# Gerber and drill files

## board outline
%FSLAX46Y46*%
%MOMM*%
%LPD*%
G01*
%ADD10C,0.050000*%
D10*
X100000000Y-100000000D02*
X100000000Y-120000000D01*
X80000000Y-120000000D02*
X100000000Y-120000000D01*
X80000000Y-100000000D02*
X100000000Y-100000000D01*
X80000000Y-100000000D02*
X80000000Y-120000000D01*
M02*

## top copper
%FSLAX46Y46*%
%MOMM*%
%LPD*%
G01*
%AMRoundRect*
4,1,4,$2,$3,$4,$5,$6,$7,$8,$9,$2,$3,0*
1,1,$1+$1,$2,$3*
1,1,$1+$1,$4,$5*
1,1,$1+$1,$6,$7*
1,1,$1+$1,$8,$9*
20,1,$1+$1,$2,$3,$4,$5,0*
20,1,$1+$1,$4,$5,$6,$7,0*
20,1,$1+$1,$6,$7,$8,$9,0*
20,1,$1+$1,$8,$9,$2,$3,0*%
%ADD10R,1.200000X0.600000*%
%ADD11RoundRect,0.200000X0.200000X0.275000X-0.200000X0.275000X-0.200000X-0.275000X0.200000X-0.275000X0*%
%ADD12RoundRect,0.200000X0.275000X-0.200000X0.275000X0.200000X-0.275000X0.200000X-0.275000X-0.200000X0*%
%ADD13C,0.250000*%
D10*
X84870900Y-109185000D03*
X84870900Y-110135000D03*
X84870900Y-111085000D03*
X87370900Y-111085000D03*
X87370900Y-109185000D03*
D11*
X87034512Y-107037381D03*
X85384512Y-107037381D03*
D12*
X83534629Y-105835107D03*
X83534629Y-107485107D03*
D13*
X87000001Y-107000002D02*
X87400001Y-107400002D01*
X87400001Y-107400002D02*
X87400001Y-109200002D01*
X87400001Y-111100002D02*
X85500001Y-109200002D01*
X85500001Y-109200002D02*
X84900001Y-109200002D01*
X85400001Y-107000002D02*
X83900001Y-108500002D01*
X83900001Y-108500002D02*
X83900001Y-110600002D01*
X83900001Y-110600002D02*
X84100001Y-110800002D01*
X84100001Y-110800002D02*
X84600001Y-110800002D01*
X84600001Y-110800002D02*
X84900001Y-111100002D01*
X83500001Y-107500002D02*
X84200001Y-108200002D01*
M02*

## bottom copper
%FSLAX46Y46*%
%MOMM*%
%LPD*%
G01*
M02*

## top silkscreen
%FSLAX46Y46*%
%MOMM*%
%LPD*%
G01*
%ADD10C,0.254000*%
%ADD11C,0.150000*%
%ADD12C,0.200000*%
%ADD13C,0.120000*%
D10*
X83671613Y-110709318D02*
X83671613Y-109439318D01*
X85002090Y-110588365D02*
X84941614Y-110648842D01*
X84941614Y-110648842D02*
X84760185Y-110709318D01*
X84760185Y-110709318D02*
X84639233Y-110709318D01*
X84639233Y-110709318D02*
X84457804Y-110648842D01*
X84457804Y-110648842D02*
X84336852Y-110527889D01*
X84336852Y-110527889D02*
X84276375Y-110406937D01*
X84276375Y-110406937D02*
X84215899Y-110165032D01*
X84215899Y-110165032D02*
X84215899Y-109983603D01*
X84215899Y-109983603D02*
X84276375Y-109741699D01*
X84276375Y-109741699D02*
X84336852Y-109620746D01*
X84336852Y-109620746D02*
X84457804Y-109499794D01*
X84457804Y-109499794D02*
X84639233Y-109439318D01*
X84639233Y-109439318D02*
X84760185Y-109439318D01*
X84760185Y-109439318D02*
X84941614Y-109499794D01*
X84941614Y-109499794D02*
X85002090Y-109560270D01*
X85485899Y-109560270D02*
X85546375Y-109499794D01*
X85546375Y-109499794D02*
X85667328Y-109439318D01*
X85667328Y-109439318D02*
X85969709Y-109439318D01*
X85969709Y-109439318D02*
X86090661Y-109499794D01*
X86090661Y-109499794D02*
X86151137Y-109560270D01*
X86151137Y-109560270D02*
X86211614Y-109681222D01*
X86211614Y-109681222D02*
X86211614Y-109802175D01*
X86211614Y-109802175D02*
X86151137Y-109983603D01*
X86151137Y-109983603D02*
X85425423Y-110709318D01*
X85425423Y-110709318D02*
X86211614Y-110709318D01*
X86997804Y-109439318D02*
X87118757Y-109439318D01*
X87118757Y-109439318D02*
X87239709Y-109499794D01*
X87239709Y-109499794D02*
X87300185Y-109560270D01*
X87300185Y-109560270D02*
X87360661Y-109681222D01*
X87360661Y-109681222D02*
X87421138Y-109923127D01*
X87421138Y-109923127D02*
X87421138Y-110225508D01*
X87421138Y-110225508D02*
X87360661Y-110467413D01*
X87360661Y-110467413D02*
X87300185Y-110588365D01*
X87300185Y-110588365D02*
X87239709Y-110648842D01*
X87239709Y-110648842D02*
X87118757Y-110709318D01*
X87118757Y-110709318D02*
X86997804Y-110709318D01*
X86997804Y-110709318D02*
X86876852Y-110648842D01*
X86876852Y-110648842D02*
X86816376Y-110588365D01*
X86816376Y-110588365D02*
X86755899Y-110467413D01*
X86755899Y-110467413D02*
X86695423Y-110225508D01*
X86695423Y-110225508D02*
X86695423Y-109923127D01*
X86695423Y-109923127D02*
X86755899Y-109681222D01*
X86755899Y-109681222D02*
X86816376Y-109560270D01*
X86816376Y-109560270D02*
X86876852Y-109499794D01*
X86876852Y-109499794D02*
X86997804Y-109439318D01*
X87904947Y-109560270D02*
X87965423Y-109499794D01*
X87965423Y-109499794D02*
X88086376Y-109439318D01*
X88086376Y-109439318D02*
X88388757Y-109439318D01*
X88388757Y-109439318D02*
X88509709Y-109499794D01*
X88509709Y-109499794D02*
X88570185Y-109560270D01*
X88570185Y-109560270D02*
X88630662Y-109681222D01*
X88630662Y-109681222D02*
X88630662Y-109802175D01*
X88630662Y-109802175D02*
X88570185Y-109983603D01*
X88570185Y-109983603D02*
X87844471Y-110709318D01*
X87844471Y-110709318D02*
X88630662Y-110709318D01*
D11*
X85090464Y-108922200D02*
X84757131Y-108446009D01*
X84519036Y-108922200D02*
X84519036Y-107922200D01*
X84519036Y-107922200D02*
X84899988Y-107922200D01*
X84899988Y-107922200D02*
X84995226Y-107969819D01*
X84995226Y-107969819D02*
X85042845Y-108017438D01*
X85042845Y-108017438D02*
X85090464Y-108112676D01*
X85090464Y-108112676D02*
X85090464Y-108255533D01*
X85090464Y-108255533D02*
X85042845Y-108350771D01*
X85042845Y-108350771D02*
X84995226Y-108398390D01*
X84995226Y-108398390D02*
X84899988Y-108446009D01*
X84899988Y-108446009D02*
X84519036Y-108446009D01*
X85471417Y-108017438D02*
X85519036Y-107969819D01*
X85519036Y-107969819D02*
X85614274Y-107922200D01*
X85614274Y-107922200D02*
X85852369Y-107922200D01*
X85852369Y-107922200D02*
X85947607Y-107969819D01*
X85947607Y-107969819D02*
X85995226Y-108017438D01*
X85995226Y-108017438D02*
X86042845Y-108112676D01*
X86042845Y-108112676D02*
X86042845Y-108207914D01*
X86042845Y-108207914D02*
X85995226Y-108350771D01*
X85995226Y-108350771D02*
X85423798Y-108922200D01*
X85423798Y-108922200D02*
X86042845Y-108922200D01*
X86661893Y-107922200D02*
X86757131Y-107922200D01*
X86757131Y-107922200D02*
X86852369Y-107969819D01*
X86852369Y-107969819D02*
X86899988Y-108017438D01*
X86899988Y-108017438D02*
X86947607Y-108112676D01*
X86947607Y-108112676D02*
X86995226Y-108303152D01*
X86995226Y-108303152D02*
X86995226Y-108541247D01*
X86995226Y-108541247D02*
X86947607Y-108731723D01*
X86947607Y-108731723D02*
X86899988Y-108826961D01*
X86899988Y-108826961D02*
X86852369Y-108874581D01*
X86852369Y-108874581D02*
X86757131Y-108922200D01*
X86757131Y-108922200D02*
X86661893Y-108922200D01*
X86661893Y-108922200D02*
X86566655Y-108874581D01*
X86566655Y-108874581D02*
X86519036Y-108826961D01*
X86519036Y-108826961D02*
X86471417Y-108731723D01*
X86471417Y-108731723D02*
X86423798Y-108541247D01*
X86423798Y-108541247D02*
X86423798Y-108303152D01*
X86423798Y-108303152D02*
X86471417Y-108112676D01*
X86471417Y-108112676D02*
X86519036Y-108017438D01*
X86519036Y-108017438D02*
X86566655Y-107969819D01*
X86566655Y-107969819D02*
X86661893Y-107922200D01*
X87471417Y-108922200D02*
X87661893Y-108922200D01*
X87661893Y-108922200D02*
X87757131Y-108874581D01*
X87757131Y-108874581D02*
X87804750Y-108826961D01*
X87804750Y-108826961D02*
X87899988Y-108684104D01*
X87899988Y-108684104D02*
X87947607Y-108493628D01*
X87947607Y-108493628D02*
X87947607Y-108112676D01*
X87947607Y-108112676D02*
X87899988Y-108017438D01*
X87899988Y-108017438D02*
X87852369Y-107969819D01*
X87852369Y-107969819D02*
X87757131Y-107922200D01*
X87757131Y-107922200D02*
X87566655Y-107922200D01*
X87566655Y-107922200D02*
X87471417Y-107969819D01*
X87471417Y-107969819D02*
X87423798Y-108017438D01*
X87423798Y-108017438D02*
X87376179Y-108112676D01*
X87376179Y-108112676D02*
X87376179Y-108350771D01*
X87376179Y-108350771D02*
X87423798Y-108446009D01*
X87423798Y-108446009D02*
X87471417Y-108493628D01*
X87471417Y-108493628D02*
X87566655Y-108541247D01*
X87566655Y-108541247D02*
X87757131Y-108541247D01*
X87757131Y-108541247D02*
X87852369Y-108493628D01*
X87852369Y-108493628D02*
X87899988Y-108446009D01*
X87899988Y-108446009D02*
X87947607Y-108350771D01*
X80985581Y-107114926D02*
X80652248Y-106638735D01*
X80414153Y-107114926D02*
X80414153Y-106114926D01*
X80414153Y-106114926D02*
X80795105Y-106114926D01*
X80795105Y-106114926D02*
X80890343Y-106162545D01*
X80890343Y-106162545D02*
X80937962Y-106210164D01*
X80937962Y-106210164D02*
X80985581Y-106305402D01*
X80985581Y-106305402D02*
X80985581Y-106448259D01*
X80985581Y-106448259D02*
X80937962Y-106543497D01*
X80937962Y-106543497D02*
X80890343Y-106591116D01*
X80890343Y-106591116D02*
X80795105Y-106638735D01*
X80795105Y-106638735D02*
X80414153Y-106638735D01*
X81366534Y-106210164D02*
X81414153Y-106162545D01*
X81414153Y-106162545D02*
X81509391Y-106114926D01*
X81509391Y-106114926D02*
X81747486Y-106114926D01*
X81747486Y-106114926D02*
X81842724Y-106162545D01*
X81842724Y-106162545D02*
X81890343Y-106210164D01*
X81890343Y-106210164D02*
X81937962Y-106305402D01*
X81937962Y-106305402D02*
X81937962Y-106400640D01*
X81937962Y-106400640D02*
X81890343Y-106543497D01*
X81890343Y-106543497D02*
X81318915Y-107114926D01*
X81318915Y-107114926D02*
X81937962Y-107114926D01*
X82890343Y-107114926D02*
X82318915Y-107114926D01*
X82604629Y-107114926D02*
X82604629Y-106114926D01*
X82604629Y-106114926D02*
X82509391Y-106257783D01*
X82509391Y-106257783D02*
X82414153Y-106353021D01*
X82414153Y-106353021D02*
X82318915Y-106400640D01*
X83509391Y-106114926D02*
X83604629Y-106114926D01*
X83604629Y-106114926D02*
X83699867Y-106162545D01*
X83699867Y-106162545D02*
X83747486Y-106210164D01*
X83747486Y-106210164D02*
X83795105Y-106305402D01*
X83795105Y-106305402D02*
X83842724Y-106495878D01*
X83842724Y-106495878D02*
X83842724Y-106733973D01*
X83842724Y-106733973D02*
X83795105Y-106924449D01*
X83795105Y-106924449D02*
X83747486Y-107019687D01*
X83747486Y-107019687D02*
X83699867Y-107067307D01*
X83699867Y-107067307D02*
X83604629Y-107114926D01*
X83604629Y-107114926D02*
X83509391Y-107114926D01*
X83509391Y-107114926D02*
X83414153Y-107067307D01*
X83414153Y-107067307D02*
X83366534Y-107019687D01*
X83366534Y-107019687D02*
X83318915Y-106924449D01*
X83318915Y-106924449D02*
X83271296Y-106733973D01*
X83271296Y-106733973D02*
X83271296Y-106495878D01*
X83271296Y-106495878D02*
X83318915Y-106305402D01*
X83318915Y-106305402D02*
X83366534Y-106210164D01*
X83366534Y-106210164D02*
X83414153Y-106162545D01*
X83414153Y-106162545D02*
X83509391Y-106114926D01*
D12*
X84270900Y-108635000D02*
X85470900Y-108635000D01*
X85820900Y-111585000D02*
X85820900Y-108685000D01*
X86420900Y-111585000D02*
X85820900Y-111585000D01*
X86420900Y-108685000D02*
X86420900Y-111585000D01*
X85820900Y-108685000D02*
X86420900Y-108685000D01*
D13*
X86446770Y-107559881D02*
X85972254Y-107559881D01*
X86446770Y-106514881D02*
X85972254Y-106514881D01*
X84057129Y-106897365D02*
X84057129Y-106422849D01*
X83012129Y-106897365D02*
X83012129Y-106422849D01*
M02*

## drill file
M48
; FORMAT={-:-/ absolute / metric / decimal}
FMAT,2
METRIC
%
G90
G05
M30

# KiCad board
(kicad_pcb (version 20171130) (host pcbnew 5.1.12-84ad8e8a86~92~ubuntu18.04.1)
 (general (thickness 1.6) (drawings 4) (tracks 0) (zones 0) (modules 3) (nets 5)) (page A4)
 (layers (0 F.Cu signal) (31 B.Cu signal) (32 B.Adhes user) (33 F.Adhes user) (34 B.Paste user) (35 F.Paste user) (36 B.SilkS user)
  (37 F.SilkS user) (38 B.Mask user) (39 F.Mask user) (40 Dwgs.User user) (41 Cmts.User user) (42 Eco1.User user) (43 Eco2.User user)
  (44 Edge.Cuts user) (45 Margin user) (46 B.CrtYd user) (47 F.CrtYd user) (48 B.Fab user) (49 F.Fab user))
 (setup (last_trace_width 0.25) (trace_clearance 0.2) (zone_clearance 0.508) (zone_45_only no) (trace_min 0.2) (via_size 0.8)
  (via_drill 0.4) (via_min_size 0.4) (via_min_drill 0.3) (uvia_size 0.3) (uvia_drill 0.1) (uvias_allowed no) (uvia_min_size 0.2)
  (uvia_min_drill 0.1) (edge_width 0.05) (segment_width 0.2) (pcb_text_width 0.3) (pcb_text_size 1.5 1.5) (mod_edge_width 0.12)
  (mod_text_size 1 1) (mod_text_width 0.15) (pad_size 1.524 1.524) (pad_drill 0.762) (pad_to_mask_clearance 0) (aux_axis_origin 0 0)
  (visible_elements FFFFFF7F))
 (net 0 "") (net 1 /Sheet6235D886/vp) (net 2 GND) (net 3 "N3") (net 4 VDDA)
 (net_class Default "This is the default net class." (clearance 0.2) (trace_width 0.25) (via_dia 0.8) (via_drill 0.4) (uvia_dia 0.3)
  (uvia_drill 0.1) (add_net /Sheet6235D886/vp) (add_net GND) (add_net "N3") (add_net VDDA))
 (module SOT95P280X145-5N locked (layer F.Cu) (at 86.120900 110.135000)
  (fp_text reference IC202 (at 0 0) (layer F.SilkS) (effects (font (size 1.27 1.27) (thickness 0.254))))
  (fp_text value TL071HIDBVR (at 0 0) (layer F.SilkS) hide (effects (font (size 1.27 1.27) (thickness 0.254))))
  (fp_line (start -1.85 -1.5) (end -0.65 -1.5) (layer F.SilkS) (width 0.2))
  (fp_line (start -0.3 1.45) (end -0.3 -1.45) (layer F.SilkS) (width 0.2))
  (fp_line (start 0.3 1.45) (end -0.3 1.45) (layer F.SilkS) (width 0.2))
  (fp_line (start 0.3 -1.45) (end 0.3 1.45) (layer F.SilkS) (width 0.2))
  (fp_line (start -0.3 -1.45) (end 0.3 -1.45) (layer F.SilkS) (width 0.2))
  (pad 1 smd rect (at -1.25 -0.95 90.000000) (size 0.6 1.2) (layers F.Cu F.Mask F.Paste) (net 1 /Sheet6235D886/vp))
  (pad 2 smd rect (at -1.25 0 90.000000) (size 0.6 1.2) (layers F.Cu F.Mask F.Paste) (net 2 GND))
  (pad 3 smd rect (at -1.25 0.95 90.000000) (size 0.6 1.2) (layers F.Cu F.Mask F.Paste) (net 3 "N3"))
  (pad 4 smd rect (at 1.25 0.95 90.000000) (size 0.6 1.2) (layers F.Cu F.Mask F.Paste) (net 1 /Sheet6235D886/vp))
  (pad 5 smd rect (at 1.25 -0.95 90.000000) (size 0.6 1.2) (layers F.Cu F.Mask F.Paste) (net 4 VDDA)))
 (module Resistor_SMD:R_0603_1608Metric (layer F.Cu) (at 86.209512 107.037381 180.000000)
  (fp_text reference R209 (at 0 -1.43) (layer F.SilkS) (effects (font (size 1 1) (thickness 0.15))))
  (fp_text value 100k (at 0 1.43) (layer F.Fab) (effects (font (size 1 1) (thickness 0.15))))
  (fp_line (start -0.237258 -0.5225) (end 0.237258 -0.5225) (layer F.SilkS) (width 0.12))
  (fp_line (start -0.237258 0.5225) (end 0.237258 0.5225) (layer F.SilkS) (width 0.12))
  (pad 1 smd roundrect (at -0.825 0 180.000000) (size 0.8 0.95) (layers F.Cu F.Mask F.Paste) (roundrect_rratio 0.25) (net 4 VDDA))
  (pad 2 smd roundrect (at 0.825 0 180.000000) (size 0.8 0.95) (layers F.Cu F.Mask F.Paste) (roundrect_rratio 0.25) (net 3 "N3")))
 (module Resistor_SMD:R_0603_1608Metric (layer F.Cu) (at 83.534629 106.660107 90.000000)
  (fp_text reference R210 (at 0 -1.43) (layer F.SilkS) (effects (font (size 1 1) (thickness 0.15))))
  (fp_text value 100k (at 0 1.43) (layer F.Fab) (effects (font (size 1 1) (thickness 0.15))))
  (fp_line (start -0.237258 0.5225) (end 0.237258 0.5225) (layer F.SilkS) (width 0.12))
  (fp_line (start -0.237258 -0.5225) (end 0.237258 -0.5225) (layer F.SilkS) (width 0.12))
  (pad 2 smd roundrect (at 0.825 0 90.000000) (size 0.8 0.95) (layers F.Cu F.Mask F.Paste) (roundrect_rratio 0.25) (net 2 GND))
  (pad 1 smd roundrect (at -0.825 0 90.000000) (size 0.8 0.95) (layers F.Cu F.Mask F.Paste) (roundrect_rratio 0.25) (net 3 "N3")))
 (gr_line (start 100 100) (end 100 120) (layer Edge.Cuts) (width 0.05))
 (gr_line (start 80 120) (end 100 120) (layer Edge.Cuts) (width 0.05))
 (gr_line (start 80 100) (end 100 100) (layer Edge.Cuts) (width 0.05))
 (gr_line (start 80 100) (end 80 120) (layer Edge.Cuts) (width 0.05))
 (segment (start 87.000001 107.000002) (end 87.400001 107.400002) (width 0.250000) (layer F.Cu) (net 4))
 (segment (start 87.400001 107.400002) (end 87.400001 109.200002) (width 0.250000) (layer F.Cu) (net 4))
 (segment (start 87.400001 111.100002) (end 85.500001 109.200002) (width 0.250000) (layer F.Cu) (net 1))
 (segment (start 85.500001 109.200002) (end 84.900001 109.200002) (width 0.250000) (layer F.Cu) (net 1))
 (segment (start 85.400001 107.000002) (end 83.900001 108.500002) (width 0.250000) (layer F.Cu) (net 3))
 (segment (start 83.900001 108.500002) (end 83.900001 110.600002) (width 0.250000) (layer F.Cu) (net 3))
 (segment (start 83.900001 110.600002) (end 84.100001 110.800002) (width 0.250000) (layer F.Cu) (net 3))
 (segment (start 84.100001 110.800002) (end 84.600001 110.800002) (width 0.250000) (layer F.Cu) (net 3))
 (segment (start 84.600001 110.800002) (end 84.900001 111.100002) (width 0.250000) (layer F.Cu) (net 3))
 (segment (start 83.500001 107.500002) (end 84.200001 108.200002) (width 0.250000) (layer F.Cu) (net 3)))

